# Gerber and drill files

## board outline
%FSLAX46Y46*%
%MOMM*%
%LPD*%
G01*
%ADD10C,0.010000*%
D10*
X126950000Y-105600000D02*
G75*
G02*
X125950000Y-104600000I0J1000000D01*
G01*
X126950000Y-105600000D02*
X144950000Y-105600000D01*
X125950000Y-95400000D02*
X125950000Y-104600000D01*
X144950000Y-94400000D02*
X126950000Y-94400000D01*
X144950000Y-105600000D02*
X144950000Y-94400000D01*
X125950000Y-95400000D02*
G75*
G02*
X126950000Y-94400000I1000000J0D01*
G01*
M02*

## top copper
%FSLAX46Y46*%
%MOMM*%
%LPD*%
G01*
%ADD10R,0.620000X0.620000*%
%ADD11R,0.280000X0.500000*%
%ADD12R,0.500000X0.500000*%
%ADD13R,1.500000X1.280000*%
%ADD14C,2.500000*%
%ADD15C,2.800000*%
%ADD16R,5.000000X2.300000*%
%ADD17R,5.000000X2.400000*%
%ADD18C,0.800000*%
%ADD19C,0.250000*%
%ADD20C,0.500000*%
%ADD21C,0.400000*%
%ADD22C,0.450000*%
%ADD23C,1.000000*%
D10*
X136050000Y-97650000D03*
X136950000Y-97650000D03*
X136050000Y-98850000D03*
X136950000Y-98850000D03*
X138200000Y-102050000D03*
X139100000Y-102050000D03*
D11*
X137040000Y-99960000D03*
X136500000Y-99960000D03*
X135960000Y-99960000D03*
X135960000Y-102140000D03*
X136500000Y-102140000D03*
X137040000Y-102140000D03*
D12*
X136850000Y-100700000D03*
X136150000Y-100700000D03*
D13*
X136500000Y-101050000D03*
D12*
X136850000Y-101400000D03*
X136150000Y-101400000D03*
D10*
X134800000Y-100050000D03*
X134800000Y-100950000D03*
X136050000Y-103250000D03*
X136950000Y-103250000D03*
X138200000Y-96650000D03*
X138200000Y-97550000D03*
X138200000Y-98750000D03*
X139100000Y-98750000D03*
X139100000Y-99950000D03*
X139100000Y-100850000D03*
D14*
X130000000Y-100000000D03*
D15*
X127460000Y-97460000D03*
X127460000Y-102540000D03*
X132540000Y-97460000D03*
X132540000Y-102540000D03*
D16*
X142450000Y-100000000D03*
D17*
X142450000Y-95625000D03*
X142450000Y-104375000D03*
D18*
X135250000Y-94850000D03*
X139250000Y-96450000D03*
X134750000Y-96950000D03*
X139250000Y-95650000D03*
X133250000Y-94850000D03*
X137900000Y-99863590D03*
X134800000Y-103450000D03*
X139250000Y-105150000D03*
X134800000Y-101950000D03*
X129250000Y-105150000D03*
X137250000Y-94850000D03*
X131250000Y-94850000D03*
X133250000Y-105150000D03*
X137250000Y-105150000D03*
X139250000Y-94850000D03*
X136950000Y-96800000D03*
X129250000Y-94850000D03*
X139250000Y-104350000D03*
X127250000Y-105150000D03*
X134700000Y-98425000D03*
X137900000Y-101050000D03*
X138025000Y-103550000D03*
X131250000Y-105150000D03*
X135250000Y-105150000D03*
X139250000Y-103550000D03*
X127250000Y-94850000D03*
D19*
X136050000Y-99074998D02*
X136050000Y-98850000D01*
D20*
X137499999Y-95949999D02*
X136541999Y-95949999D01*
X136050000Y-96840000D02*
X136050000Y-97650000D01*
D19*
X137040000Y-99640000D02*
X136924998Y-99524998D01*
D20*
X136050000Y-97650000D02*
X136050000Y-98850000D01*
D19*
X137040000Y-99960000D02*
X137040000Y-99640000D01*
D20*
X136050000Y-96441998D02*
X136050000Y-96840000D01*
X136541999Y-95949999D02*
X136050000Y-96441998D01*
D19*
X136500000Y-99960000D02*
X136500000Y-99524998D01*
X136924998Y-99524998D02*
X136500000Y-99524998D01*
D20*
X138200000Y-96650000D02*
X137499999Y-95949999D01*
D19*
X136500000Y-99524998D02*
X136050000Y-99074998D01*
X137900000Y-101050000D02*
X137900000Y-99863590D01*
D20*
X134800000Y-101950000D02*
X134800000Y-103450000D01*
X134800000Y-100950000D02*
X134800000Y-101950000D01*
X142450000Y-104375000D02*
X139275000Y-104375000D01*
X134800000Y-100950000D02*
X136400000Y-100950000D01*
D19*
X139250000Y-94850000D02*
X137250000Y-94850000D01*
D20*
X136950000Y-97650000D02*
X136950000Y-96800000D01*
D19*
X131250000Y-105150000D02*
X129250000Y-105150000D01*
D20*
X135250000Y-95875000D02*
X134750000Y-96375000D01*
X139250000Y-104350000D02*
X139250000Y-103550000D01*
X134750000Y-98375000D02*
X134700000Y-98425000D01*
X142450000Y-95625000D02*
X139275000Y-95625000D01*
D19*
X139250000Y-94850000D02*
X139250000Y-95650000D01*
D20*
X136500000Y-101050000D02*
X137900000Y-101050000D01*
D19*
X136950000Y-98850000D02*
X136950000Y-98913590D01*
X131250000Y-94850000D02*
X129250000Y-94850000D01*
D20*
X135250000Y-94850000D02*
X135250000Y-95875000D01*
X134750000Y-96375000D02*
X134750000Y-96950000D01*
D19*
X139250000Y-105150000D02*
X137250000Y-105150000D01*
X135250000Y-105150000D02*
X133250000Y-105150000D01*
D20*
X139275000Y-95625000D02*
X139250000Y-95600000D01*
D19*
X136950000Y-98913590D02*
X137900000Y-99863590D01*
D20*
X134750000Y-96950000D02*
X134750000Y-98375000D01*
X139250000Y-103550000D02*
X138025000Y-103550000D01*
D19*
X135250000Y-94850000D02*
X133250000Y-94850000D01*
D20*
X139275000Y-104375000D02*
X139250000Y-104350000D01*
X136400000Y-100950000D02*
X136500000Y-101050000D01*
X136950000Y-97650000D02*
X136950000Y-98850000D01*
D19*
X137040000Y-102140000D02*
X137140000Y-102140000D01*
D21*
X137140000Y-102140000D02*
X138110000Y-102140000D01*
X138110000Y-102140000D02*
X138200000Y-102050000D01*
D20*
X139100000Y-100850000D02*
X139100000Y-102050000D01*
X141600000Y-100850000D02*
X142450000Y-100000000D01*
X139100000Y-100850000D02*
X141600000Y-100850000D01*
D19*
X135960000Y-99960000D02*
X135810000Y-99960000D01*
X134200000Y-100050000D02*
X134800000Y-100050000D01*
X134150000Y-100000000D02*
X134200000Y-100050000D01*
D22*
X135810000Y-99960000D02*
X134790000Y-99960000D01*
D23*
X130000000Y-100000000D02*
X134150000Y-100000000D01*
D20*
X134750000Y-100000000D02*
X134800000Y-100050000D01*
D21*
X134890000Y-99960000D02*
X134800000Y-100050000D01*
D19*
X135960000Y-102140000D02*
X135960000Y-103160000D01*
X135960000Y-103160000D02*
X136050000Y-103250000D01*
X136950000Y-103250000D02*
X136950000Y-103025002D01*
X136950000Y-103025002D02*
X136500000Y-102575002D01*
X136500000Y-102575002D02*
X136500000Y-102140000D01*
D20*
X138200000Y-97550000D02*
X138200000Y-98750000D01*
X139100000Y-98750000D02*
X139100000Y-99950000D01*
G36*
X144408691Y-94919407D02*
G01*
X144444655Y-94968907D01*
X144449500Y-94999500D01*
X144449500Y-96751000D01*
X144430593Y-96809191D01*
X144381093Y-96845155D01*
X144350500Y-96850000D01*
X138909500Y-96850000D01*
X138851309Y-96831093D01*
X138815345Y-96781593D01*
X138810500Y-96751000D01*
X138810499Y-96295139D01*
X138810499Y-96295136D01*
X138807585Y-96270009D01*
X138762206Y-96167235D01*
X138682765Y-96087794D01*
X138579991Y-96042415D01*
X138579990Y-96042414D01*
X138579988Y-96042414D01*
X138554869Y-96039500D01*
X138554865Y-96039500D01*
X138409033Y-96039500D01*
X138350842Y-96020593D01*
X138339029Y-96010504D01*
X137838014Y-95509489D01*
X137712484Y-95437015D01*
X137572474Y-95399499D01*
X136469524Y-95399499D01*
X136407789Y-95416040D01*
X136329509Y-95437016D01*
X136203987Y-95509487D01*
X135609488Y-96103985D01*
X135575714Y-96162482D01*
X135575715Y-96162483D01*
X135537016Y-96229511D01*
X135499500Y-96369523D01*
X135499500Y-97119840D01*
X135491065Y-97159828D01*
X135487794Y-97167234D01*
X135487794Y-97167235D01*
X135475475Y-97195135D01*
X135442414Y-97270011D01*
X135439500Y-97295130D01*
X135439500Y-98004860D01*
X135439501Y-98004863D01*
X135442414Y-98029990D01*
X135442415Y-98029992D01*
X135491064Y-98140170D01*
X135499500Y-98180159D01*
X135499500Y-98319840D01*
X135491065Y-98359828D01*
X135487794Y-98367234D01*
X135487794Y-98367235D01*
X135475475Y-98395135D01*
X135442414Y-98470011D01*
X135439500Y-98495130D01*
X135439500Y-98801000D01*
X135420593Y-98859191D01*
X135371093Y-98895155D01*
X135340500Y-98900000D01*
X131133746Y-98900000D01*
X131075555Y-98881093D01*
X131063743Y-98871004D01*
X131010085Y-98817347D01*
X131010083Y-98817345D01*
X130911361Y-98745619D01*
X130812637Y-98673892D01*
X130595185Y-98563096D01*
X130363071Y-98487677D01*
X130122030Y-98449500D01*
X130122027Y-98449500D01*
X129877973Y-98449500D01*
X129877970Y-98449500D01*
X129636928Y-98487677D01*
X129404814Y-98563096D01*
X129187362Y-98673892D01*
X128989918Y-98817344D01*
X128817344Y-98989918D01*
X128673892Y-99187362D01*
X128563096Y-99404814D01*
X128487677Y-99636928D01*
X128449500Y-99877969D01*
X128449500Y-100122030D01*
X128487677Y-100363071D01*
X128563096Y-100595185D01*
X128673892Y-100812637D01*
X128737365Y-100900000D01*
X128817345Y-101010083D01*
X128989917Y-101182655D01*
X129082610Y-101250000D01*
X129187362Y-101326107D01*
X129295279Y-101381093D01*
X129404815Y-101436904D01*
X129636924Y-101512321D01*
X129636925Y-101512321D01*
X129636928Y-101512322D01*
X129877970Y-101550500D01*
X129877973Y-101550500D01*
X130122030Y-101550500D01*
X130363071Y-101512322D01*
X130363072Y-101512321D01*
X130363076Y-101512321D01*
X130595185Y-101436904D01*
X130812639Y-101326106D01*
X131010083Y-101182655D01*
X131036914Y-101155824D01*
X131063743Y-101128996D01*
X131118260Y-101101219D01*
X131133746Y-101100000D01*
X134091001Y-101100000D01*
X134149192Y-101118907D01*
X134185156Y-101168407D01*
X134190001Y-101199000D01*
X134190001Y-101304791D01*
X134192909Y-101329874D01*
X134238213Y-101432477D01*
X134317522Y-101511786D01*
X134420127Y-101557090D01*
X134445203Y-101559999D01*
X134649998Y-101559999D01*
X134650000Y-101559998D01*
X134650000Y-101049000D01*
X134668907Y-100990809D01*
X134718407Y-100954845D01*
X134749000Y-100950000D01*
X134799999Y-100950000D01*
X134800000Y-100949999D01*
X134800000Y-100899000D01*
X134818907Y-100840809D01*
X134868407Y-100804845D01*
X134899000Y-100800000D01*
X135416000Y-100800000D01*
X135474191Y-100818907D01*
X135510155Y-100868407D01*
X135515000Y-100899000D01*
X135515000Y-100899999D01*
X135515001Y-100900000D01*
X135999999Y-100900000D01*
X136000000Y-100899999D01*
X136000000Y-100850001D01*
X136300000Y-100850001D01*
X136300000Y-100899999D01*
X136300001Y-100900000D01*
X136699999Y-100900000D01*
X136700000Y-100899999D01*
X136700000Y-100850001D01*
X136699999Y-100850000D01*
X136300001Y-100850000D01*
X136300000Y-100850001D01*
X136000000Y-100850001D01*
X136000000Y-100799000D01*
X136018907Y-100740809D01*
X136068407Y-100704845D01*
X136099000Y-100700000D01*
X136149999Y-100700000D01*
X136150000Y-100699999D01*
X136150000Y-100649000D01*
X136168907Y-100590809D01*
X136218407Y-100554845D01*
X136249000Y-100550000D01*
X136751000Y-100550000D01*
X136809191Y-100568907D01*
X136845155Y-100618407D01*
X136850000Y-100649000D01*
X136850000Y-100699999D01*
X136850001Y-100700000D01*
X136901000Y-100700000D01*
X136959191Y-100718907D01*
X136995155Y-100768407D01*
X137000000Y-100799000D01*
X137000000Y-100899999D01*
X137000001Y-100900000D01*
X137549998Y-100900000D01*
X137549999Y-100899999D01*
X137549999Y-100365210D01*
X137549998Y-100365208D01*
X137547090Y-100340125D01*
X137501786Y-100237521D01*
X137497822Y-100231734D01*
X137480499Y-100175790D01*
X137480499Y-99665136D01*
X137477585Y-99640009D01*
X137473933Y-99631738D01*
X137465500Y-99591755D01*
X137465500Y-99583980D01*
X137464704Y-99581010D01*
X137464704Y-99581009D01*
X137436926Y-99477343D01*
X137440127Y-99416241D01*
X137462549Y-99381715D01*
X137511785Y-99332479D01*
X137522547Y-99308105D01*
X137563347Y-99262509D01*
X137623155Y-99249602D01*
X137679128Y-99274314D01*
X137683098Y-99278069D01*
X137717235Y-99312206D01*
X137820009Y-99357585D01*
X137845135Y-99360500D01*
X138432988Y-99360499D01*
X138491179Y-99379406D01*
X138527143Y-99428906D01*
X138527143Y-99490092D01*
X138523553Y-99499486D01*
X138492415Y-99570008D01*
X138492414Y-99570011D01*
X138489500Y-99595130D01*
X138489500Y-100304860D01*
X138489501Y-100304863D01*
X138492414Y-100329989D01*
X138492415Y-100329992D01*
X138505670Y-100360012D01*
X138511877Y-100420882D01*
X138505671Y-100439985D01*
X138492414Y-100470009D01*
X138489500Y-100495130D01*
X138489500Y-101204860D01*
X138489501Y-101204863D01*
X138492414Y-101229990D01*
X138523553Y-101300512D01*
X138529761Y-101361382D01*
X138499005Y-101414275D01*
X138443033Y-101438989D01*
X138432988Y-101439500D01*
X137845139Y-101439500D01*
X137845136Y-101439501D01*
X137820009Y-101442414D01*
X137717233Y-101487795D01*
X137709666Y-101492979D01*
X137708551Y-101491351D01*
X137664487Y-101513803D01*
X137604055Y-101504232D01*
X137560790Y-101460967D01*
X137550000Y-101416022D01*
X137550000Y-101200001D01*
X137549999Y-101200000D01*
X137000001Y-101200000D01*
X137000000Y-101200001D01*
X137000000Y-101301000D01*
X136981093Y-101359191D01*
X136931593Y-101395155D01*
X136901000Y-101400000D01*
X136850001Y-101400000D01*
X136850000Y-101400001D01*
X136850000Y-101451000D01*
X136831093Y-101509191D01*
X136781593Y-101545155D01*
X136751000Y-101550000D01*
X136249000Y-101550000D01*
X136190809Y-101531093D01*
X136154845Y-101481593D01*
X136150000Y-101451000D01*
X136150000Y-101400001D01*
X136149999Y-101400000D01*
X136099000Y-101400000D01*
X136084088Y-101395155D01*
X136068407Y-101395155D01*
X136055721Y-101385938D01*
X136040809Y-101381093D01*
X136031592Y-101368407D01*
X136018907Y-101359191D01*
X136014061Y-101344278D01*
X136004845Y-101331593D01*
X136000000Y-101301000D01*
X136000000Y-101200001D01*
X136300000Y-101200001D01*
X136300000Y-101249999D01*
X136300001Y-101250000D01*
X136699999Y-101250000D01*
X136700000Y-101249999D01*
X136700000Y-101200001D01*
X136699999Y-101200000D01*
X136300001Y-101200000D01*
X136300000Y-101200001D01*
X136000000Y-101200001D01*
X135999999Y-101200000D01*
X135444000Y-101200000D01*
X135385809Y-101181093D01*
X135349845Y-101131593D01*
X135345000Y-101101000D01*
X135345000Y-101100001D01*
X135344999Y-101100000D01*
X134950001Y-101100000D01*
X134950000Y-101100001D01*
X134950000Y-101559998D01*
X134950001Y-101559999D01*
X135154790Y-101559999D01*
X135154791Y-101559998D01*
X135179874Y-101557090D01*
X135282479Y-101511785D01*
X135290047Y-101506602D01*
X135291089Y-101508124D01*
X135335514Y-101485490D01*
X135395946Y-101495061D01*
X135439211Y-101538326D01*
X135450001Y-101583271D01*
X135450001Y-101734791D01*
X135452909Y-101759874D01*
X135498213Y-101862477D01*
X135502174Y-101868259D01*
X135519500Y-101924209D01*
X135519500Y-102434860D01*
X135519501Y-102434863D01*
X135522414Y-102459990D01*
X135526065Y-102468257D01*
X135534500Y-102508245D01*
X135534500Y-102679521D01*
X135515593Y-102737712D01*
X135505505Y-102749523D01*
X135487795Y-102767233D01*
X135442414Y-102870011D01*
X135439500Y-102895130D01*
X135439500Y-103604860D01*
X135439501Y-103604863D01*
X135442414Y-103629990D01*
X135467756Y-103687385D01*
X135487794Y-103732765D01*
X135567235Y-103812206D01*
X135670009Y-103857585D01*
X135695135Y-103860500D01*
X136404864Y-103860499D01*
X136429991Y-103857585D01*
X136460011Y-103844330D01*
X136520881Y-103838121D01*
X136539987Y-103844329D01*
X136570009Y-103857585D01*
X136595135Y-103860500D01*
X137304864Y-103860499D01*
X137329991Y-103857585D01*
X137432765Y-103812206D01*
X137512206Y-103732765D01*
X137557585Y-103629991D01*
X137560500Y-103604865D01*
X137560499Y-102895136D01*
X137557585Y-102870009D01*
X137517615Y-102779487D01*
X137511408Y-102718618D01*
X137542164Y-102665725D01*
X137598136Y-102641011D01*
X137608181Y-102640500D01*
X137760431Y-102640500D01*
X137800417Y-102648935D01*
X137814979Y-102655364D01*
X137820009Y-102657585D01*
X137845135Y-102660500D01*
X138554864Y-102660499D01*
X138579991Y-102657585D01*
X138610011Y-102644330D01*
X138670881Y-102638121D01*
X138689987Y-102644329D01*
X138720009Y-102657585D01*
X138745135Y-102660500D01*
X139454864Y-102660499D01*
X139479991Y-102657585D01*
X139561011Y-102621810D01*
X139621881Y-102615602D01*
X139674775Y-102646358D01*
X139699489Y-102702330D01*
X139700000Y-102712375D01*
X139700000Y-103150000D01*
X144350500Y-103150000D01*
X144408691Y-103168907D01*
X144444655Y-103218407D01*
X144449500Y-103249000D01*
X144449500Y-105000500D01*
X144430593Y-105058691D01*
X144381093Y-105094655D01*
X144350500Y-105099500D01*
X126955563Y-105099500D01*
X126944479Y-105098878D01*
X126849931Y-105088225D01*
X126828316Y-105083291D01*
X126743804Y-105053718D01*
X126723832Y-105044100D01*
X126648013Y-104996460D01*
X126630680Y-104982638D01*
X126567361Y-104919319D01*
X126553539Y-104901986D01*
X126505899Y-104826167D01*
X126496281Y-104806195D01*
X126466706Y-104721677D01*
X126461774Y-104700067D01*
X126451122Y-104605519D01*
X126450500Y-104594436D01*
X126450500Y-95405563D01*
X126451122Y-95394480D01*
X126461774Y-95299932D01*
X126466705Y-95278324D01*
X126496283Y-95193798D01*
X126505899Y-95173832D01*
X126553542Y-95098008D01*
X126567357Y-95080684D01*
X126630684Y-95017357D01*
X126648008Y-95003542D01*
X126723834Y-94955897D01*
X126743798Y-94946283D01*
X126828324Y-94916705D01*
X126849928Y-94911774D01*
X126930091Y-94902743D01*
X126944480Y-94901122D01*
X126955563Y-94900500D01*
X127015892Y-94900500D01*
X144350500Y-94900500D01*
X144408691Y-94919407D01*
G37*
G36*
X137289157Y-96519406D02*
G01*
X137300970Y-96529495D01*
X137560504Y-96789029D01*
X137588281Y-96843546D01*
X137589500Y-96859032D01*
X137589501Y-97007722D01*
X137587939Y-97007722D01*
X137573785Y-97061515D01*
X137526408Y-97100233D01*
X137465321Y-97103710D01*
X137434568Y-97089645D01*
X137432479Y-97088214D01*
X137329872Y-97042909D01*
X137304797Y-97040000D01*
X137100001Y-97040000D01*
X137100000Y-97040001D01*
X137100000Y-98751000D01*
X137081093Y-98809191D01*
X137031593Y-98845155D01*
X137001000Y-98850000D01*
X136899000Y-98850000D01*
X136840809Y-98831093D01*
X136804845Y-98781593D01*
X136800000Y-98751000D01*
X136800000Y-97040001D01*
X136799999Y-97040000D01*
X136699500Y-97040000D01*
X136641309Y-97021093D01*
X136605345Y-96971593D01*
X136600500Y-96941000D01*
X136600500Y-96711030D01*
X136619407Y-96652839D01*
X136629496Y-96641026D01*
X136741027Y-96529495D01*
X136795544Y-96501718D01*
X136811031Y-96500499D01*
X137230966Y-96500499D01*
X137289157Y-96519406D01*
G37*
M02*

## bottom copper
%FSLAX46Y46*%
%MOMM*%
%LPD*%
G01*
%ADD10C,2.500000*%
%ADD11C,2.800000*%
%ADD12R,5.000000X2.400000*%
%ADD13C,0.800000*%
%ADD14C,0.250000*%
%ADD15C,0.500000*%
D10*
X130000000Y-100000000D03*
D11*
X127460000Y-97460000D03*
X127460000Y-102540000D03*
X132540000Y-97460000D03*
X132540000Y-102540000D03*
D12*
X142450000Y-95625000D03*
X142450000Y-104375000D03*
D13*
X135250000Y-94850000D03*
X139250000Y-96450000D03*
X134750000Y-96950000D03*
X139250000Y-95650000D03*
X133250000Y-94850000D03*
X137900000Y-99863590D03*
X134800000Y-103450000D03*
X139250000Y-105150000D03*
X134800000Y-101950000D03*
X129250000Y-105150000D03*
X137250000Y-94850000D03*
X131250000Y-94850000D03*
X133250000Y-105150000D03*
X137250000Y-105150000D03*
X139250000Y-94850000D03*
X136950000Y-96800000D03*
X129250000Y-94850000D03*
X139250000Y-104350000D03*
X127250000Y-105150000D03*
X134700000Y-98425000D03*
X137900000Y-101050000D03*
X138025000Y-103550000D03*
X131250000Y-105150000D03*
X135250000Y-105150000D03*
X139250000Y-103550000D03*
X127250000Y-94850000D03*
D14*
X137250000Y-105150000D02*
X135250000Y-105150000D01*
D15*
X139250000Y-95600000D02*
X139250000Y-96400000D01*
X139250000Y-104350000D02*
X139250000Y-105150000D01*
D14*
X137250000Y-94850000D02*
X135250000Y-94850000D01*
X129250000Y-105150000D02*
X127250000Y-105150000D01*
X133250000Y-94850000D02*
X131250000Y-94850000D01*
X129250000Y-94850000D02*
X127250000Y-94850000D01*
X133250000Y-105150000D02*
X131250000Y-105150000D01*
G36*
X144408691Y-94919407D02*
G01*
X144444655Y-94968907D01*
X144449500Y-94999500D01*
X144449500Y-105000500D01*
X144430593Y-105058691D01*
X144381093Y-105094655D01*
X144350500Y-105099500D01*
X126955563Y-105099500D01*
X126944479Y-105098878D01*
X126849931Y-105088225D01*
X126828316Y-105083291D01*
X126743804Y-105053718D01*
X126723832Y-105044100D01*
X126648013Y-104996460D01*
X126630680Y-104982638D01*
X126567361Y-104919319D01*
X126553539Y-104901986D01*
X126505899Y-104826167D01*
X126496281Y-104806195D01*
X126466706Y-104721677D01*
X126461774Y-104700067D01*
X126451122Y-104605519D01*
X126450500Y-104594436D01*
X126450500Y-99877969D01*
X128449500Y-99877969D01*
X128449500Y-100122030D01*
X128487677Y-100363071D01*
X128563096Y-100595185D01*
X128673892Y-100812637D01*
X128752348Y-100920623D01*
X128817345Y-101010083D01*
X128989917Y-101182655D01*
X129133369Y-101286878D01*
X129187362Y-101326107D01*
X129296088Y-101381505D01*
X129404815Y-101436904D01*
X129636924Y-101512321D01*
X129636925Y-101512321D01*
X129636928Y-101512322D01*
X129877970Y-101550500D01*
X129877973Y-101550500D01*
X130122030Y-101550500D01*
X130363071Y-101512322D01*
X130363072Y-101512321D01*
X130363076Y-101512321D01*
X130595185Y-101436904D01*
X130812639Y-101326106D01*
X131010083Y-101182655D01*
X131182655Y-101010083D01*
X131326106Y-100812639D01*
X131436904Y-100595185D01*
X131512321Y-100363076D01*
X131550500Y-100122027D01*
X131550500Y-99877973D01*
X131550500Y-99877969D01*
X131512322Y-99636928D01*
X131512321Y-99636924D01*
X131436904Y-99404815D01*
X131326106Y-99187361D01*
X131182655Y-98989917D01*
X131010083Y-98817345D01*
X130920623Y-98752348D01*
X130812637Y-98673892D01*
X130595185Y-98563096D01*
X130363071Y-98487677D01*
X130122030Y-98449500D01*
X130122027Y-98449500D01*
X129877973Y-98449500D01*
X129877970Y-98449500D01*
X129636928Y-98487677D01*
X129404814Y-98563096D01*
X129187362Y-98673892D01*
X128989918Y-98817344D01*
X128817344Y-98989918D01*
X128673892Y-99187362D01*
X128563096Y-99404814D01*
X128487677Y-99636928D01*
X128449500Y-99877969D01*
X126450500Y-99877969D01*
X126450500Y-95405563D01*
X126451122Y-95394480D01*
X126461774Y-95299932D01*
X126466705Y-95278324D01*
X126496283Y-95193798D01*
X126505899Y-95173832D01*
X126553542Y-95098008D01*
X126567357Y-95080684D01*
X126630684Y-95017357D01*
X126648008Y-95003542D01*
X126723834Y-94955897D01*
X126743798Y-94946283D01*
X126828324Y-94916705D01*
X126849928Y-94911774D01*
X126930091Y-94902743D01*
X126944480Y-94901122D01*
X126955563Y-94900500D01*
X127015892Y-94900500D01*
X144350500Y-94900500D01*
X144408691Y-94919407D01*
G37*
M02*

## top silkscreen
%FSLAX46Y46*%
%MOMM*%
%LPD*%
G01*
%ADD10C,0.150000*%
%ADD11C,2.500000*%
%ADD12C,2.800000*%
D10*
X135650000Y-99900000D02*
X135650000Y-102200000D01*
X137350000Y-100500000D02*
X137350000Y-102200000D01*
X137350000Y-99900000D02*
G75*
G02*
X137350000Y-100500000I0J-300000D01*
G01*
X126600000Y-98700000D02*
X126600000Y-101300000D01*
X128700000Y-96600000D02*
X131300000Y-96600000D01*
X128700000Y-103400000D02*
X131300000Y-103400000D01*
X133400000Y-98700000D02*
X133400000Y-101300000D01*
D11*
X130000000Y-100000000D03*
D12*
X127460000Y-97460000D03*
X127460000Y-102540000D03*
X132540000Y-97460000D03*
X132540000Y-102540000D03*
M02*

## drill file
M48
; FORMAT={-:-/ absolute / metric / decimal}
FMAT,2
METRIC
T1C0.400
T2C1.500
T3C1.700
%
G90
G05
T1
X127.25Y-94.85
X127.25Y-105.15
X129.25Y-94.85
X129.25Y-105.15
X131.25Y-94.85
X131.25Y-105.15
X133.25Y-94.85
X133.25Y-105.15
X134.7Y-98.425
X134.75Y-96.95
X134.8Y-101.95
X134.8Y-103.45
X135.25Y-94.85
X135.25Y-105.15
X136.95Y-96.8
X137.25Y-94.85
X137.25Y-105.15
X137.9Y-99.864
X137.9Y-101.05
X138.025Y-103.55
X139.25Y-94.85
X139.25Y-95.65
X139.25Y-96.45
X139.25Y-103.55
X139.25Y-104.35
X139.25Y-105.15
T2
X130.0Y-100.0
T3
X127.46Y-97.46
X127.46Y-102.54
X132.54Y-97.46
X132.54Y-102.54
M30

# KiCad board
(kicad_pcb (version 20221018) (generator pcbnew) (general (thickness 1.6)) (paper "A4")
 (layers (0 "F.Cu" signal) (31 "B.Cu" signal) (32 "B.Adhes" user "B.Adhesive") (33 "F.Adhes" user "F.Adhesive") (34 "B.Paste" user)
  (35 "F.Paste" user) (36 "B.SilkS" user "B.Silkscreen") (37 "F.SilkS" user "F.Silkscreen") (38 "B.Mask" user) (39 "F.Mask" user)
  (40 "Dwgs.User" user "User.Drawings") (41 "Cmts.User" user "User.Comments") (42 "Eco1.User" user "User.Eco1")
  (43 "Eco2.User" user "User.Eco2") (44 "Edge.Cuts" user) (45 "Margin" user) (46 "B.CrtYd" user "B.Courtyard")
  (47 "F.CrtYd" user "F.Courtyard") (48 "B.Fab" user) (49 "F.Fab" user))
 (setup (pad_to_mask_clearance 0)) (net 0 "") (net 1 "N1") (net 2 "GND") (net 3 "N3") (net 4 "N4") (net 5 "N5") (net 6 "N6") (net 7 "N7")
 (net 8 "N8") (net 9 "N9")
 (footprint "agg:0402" (layer "F.Cu") (at 136.5 97.65)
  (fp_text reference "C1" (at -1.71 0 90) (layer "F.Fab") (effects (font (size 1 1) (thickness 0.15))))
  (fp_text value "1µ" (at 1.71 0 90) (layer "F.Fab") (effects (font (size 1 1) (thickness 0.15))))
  (pad "1" smd rect (at -0.45 0) (size 0.62 0.62) (layers "F.Cu" "F.Paste" "F.Mask") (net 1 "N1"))
  (pad "2" smd rect (at 0.45 0) (size 0.62 0.62) (layers "F.Cu" "F.Paste" "F.Mask") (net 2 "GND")))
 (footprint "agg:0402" (layer "F.Cu") (at 136.5 98.85)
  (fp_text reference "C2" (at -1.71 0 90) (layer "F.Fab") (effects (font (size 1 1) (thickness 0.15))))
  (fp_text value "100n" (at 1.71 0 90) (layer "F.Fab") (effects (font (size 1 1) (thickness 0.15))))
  (pad "1" smd rect (at -0.45 0) (size 0.62 0.62) (layers "F.Cu" "F.Paste" "F.Mask") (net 1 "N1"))
  (pad "2" smd rect (at 0.45 0) (size 0.62 0.62) (layers "F.Cu" "F.Paste" "F.Mask") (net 2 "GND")))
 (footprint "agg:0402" (layer "F.Cu") (at 138.65 102.05)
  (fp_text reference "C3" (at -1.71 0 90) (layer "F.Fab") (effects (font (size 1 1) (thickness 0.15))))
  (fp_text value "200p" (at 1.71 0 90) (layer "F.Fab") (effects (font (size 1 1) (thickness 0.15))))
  (pad "1" smd rect (at -0.45 0) (size 0.62 0.62) (layers "F.Cu" "F.Paste" "F.Mask") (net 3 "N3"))
  (pad "2" smd rect (at 0.45 0) (size 0.62 0.62) (layers "F.Cu" "F.Paste" "F.Mask") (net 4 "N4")))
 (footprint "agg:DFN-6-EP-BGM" (layer "F.Cu") (at 136.5 101.05 -90)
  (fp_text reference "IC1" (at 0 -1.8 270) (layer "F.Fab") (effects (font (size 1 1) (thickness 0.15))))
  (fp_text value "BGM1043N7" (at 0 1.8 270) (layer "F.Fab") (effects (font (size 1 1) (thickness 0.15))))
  (fp_line (start -1.15 0.85) (end 1.15 0.85) (stroke (width 0.15) (type solid)) (layer "F.SilkS"))
  (fp_line (start -0.55 -0.85) (end 1.15 -0.85) (stroke (width 0.15) (type solid)) (layer "F.SilkS"))
  (fp_arc (start -1.15 -0.85) (mid -0.85 -1.15) (end -0.55 -0.85) (stroke (width 0.15) (type solid)) (layer "F.SilkS"))
  (pad "1" smd rect (at -1.09 -0.54 270) (size 0.5 0.28) (layers "F.Cu" "F.Paste" "F.Mask") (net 1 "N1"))
  (pad "2" smd rect (at -1.09 0 270) (size 0.5 0.28) (layers "F.Cu" "F.Paste" "F.Mask") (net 1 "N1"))
  (pad "3" smd rect (at -1.09 0.54 270) (size 0.5 0.28) (layers "F.Cu" "F.Paste" "F.Mask") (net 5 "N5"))
  (pad "4" smd rect (at 1.09 0.54 270) (size 0.5 0.28) (layers "F.Cu" "F.Paste" "F.Mask") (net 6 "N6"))
  (pad "5" smd rect (at 1.09 0 270) (size 0.5 0.28) (layers "F.Cu" "F.Paste" "F.Mask") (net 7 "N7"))
  (pad "6" smd rect (at 1.09 -0.54 270) (size 0.5 0.28) (layers "F.Cu" "F.Paste" "F.Mask") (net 3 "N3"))
  (pad "EP" smd rect (at -0.35 -0.35 270) (size 0.5 0.5) (layers "F.Cu" "F.Paste") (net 2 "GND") (solder_paste_margin 0.001))
  (pad "EP" smd rect (at -0.35 0.35 270) (size 0.5 0.5) (layers "F.Cu" "F.Paste") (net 2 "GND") (solder_paste_margin 0.001))
  (pad "EP" smd rect (at 0 0 270) (size 1.28 1.5) (layers "F.Cu" "F.Mask") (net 2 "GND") (solder_mask_margin 0.001))
  (pad "EP" smd rect (at 0.35 -0.35 270) (size 0.5 0.5) (layers "F.Cu" "F.Paste") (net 2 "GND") (solder_paste_margin 0.001))
  (pad "EP" smd rect (at 0.35 0.35 270) (size 0.5 0.5) (layers "F.Cu" "F.Paste") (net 2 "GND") (solder_paste_margin 0.001)))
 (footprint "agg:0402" (layer "F.Cu") (at 134.8 100.5 -90)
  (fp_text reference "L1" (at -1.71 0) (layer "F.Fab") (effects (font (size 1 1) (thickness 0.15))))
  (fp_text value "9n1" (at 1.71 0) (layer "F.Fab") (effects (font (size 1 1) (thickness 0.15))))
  (pad "1" smd rect (at -0.45 0 270) (size 0.62 0.62) (layers "F.Cu" "F.Paste" "F.Mask") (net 5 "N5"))
  (pad "2" smd rect (at 0.45 0 270) (size 0.62 0.62) (layers "F.Cu" "F.Paste" "F.Mask") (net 2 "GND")))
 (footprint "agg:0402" (layer "F.Cu") (at 136.5 103.25)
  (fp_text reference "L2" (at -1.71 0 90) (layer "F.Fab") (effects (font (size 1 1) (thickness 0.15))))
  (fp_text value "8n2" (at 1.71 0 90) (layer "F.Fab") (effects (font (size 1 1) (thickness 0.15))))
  (pad "1" smd rect (at -0.45 0) (size 0.62 0.62) (layers "F.Cu" "F.Paste" "F.Mask") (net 6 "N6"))
  (pad "2" smd rect (at 0.45 0) (size 0.62 0.62) (layers "F.Cu" "F.Paste" "F.Mask") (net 7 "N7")))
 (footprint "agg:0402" (layer "F.Cu") (at 138.2 97.1 -90)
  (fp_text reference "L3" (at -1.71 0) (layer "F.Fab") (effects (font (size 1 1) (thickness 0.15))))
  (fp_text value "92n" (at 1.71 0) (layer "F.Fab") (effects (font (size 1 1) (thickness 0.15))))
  (pad "1" smd rect (at -0.45 0 270) (size 0.62 0.62) (layers "F.Cu" "F.Paste" "F.Mask") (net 1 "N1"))
  (pad "2" smd rect (at 0.45 0 270) (size 0.62 0.62) (layers "F.Cu" "F.Paste" "F.Mask") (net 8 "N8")))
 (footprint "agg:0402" (layer "F.Cu") (at 138.65 98.75)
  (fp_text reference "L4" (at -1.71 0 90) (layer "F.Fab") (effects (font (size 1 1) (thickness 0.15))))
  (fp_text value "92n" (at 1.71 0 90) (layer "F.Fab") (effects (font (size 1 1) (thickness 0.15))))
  (pad "1" smd rect (at -0.45 0) (size 0.62 0.62) (layers "F.Cu" "F.Paste" "F.Mask") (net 8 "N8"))
  (pad "2" smd rect (at 0.45 0) (size 0.62 0.62) (layers "F.Cu" "F.Paste" "F.Mask") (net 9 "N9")))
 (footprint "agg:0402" (layer "F.Cu") (at 139.1 100.4 -90)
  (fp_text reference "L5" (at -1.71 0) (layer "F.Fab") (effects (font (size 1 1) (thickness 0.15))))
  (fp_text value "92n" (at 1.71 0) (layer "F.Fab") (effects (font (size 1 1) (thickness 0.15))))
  (pad "1" smd rect (at -0.45 0 270) (size 0.62 0.62) (layers "F.Cu" "F.Paste" "F.Mask") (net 9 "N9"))
  (pad "2" smd rect (at 0.45 0 270) (size 0.62 0.62) (layers "F.Cu" "F.Paste" "F.Mask") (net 4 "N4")))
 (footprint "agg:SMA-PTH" (layer "F.Cu") (at 130 100)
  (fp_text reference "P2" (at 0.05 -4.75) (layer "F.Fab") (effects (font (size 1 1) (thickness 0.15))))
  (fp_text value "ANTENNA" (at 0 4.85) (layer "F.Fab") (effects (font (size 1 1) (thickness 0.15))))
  (fp_line (start -3.4 -1.3) (end -3.4 1.3) (stroke (width 0.15) (type solid)) (layer "F.SilkS"))
  (fp_line (start -1.3 -3.4) (end 1.3 -3.4) (stroke (width 0.15) (type solid)) (layer "F.SilkS"))
  (fp_line (start -1.3 3.4) (end 1.3 3.4) (stroke (width 0.15) (type solid)) (layer "F.SilkS"))
  (fp_line (start 3.4 -1.3) (end 3.4 1.3) (stroke (width 0.15) (type solid)) (layer "F.SilkS"))
  (pad "1" thru_hole circle (at 0 0) (size 2.5 2.5) (drill 1.5) (layers "*.Cu" "*.Mask" "F.SilkS") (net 5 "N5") (zone_connect 2))
  (pad "2" thru_hole circle (at -2.54 -2.54) (size 2.8 2.8) (drill 1.7) (layers "*.Cu" "*.Mask" "F.SilkS") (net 2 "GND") (zone_connect 2))
  (pad "2" thru_hole circle (at -2.54 2.54) (size 2.8 2.8) (drill 1.7) (layers "*.Cu" "*.Mask" "F.SilkS") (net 2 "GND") (zone_connect 2))
  (pad "2" thru_hole circle (at 2.54 -2.54) (size 2.8 2.8) (drill 1.7) (layers "*.Cu" "*.Mask" "F.SilkS") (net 2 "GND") (zone_connect 2))
  (pad "2" thru_hole circle (at 2.54 2.54) (size 2.8 2.8) (drill 1.7) (layers "*.Cu" "*.Mask" "F.SilkS") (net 2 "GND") (zone_connect 2)))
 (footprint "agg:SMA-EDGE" (layer "F.Cu") (at 142.45 100 -90)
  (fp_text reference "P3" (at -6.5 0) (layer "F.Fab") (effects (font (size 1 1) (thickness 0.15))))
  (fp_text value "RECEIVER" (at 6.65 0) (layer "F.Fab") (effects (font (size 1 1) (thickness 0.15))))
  (pad "1" smd rect (at 0 0 270) (size 2.3 5) (layers "F.Cu" "F.Paste" "F.Mask") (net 4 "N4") (zone_connect 2))
  (pad "2" smd rect (at -4.375 0 270) (size 2.4 5) (layers "F.Cu" "F.Paste" "F.Mask") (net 2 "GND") (zone_connect 2))
  (pad "2" smd rect (at -4.375 0 270) (size 2.4 5) (layers "B.Cu" "B.Paste" "B.Mask") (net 2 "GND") (zone_connect 2))
  (pad "2" smd rect (at 4.375 0 270) (size 2.4 5) (layers "F.Cu" "F.Paste" "F.Mask") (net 2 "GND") (zone_connect 2))
  (pad "2" smd rect (at 4.375 0 270) (size 2.4 5) (layers "B.Cu" "B.Paste" "B.Mask") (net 2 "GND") (zone_connect 2)))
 (gr_arc (start 126.95 105.6) (mid 126.242893 105.307107) (end 125.95 104.6) (stroke (width 0.01) (type solid)) (layer "Edge.Cuts"))
 (gr_line (start 126.95 105.6) (end 144.95 105.6) (stroke (width 0.01) (type solid)) (layer "Edge.Cuts"))
 (gr_line (start 125.95 95.4) (end 125.95 104.6) (stroke (width 0.01) (type solid)) (layer "Edge.Cuts"))
 (gr_line (start 144.95 94.4) (end 126.95 94.4) (stroke (width 0.01) (type solid)) (layer "Edge.Cuts"))
 (gr_line (start 144.95 105.6) (end 144.95 94.4) (stroke (width 0.01) (type solid)) (layer "Edge.Cuts"))
 (gr_arc (start 125.95 95.4) (mid 126.242893 94.692893) (end 126.95 94.4) (stroke (width 0.01) (type solid)) (layer "Edge.Cuts"))
 (segment (start 136.05 99.074998) (end 136.05 98.85) (width 0.25) (layer "F.Cu") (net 1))
 (segment (start 137.499999 95.949999) (end 136.541999 95.949999) (width 0.5) (layer "F.Cu") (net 1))
 (segment (start 136.05 96.84) (end 136.05 97.65) (width 0.5) (layer "F.Cu") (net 1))
 (segment (start 137.04 99.64) (end 136.924998 99.524998) (width 0.25) (layer "F.Cu") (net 1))
 (segment (start 136.05 97.65) (end 136.05 98.85) (width 0.5) (layer "F.Cu") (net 1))
 (segment (start 137.04 99.96) (end 137.04 99.64) (width 0.25) (layer "F.Cu") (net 1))
 (segment (start 136.05 96.441998) (end 136.05 96.84) (width 0.5) (layer "F.Cu") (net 1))
 (segment (start 136.541999 95.949999) (end 136.05 96.441998) (width 0.5) (layer "F.Cu") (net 1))
 (segment (start 136.5 99.96) (end 136.5 99.524998) (width 0.25) (layer "F.Cu") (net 1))
 (segment (start 136.924998 99.524998) (end 136.5 99.524998) (width 0.25) (layer "F.Cu") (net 1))
 (segment (start 138.2 96.65) (end 137.499999 95.949999) (width 0.5) (layer "F.Cu") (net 1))
 (segment (start 136.5 99.524998) (end 136.05 99.074998) (width 0.25) (layer "F.Cu") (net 1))
 (segment (start 137.9 101.05) (end 137.9 99.86359) (width 0.25) (layer "F.Cu") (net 2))
 (segment (start 134.8 101.95) (end 134.8 103.45) (width 0.5) (layer "F.Cu") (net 2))
 (segment (start 134.8 100.95) (end 134.8 101.95) (width 0.5) (layer "F.Cu") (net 2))
 (segment (start 142.45 104.375) (end 139.275 104.375) (width 0.5) (layer "F.Cu") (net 2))
 (segment (start 134.8 100.95) (end 136.4 100.95) (width 0.5) (layer "F.Cu") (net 2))
 (segment (start 139.25 94.85) (end 137.25 94.85) (width 0.25) (layer "F.Cu") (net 2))
 (segment (start 136.95 97.65) (end 136.95 96.8) (width 0.5) (layer "F.Cu") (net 2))
 (segment (start 131.25 105.15) (end 129.25 105.15) (width 0.25) (layer "F.Cu") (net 2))
 (segment (start 135.25 95.875) (end 134.75 96.375) (width 0.5) (layer "F.Cu") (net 2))
 (segment (start 139.25 104.35) (end 139.25 103.55) (width 0.5) (layer "F.Cu") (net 2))
 (segment (start 134.75 98.375) (end 134.7 98.425) (width 0.5) (layer "F.Cu") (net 2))
 (segment (start 142.45 95.625) (end 139.275 95.625) (width 0.5) (layer "F.Cu") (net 2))
 (segment (start 139.25 94.85) (end 139.25 95.65) (width 0.25) (layer "F.Cu") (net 2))
 (segment (start 136.5 101.05) (end 137.9 101.05) (width 0.5) (layer "F.Cu") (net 2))
 (segment (start 136.95 98.85) (end 136.95 98.91359) (width 0.25) (layer "F.Cu") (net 2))
 (segment (start 131.25 94.85) (end 129.25 94.85) (width 0.25) (layer "F.Cu") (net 2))
 (segment (start 135.25 94.85) (end 135.25 95.875) (width 0.5) (layer "F.Cu") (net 2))
 (segment (start 134.75 96.375) (end 134.75 96.95) (width 0.5) (layer "F.Cu") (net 2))
 (segment (start 139.25 105.15) (end 137.25 105.15) (width 0.25) (layer "F.Cu") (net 2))
 (segment (start 135.25 105.15) (end 133.25 105.15) (width 0.25) (layer "F.Cu") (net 2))
 (segment (start 139.275 95.625) (end 139.25 95.6) (width 0.5) (layer "F.Cu") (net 2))
 (segment (start 136.95 98.91359) (end 137.9 99.86359) (width 0.25) (layer "F.Cu") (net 2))
 (segment (start 134.75 96.95) (end 134.75 98.375) (width 0.5) (layer "F.Cu") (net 2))
 (segment (start 139.25 103.55) (end 138.025 103.55) (width 0.5) (layer "F.Cu") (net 2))
 (segment (start 135.25 94.85) (end 133.25 94.85) (width 0.25) (layer "F.Cu") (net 2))
 (segment (start 139.275 104.375) (end 139.25 104.35) (width 0.5) (layer "F.Cu") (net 2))
 (segment (start 136.4 100.95) (end 136.5 101.05) (width 0.5) (layer "F.Cu") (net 2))
 (segment (start 136.95 97.65) (end 136.95 98.85) (width 0.5) (layer "F.Cu") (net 2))
 (via (at 135.25 94.85) (size 0.8) (drill 0.4) (layers "F.Cu" "B.Cu") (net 2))
 (via (at 139.25 96.45) (size 0.8) (drill 0.4) (layers "F.Cu" "B.Cu") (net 2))
 (via (at 134.75 96.95) (size 0.8) (drill 0.4) (layers "F.Cu" "B.Cu") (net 2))
 (via (at 139.25 95.65) (size 0.8) (drill 0.4) (layers "F.Cu" "B.Cu") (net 2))
 (via (at 133.25 94.85) (size 0.8) (drill 0.4) (layers "F.Cu" "B.Cu") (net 2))
 (via (at 137.9 99.86359) (size 0.8) (drill 0.4) (layers "F.Cu" "B.Cu") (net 2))
 (via (at 134.8 103.45) (size 0.8) (drill 0.4) (layers "F.Cu" "B.Cu") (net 2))
 (via (at 139.25 105.15) (size 0.8) (drill 0.4) (layers "F.Cu" "B.Cu") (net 2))
 (via (at 134.8 101.95) (size 0.8) (drill 0.4) (layers "F.Cu" "B.Cu") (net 2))
 (via (at 129.25 105.15) (size 0.8) (drill 0.4) (layers "F.Cu" "B.Cu") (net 2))
 (via (at 137.25 94.85) (size 0.8) (drill 0.4) (layers "F.Cu" "B.Cu") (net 2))
 (via (at 131.25 94.85) (size 0.8) (drill 0.4) (layers "F.Cu" "B.Cu") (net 2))
 (via (at 133.25 105.15) (size 0.8) (drill 0.4) (layers "F.Cu" "B.Cu") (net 2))
 (via (at 137.25 105.15) (size 0.8) (drill 0.4) (layers "F.Cu" "B.Cu") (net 2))
 (via (at 139.25 94.85) (size 0.8) (drill 0.4) (layers "F.Cu" "B.Cu") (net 2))
 (via (at 136.95 96.8) (size 0.8) (drill 0.4) (layers "F.Cu" "B.Cu") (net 2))
 (via (at 129.25 94.85) (size 0.8) (drill 0.4) (layers "F.Cu" "B.Cu") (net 2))
 (via (at 139.25 104.35) (size 0.8) (drill 0.4) (layers "F.Cu" "B.Cu") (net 2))
 (via (at 127.25 105.15) (size 0.8) (drill 0.4) (layers "F.Cu" "B.Cu") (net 2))
 (via (at 134.7 98.425) (size 0.8) (drill 0.4) (layers "F.Cu" "B.Cu") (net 2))
 (via (at 137.9 101.05) (size 0.8) (drill 0.4) (layers "F.Cu" "B.Cu") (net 2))
 (via (at 138.025 103.55) (size 0.8) (drill 0.4) (layers "F.Cu" "B.Cu") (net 2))
 (via (at 131.25 105.15) (size 0.8) (drill 0.4) (layers "F.Cu" "B.Cu") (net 2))
 (via (at 135.25 105.15) (size 0.8) (drill 0.4) (layers "F.Cu" "B.Cu") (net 2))
 (via (at 139.25 103.55) (size 0.8) (drill 0.4) (layers "F.Cu" "B.Cu") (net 2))
 (via (at 127.25 94.85) (size 0.8) (drill 0.4) (layers "F.Cu" "B.Cu") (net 2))
 (segment (start 137.25 105.15) (end 135.25 105.15) (width 0.25) (layer "B.Cu") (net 2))
 (segment (start 139.25 95.6) (end 139.25 96.4) (width 0.5) (layer "B.Cu") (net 2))
 (segment (start 139.25 104.35) (end 139.25 105.15) (width 0.5) (layer "B.Cu") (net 2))
 (segment (start 137.25 94.85) (end 135.25 94.85) (width 0.25) (layer "B.Cu") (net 2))
 (segment (start 129.25 105.15) (end 127.25 105.15) (width 0.25) (layer "B.Cu") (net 2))
 (segment (start 133.25 94.85) (end 131.25 94.85) (width 0.25) (layer "B.Cu") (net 2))
 (segment (start 129.25 94.85) (end 127.25 94.85) (width 0.25) (layer "B.Cu") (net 2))
 (segment (start 133.25 105.15) (end 131.25 105.15) (width 0.25) (layer "B.Cu") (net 2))
 (segment (start 137.04 102.14) (end 137.14 102.14) (width 0.25) (layer "F.Cu") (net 3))
 (segment (start 137.14 102.14) (end 138.11 102.14) (width 0.4) (layer "F.Cu") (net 3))
 (segment (start 138.11 102.14) (end 138.2 102.05) (width 0.4) (layer "F.Cu") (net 3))
 (segment (start 139.1 100.85) (end 139.1 102.05) (width 0.5) (layer "F.Cu") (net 4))
 (segment (start 141.6 100.85) (end 142.45 100) (width 0.5) (layer "F.Cu") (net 4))
 (segment (start 139.1 100.85) (end 141.6 100.85) (width 0.5) (layer "F.Cu") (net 4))
 (segment (start 135.96 99.96) (end 135.81 99.96) (width 0.25) (layer "F.Cu") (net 5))
 (segment (start 134.2 100.05) (end 134.8 100.05) (width 0.25) (layer "F.Cu") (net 5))
 (segment (start 134.15 100) (end 134.2 100.05) (width 0.25) (layer "F.Cu") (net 5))
 (segment (start 135.81 99.96) (end 134.79 99.96) (width 0.45) (layer "F.Cu") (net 5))
 (segment (start 130 100) (end 134.15 100) (width 1) (layer "F.Cu") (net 5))
 (segment (start 134.75 100) (end 134.8 100.05) (width 0.5) (layer "F.Cu") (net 5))
 (segment (start 134.89 99.96) (end 134.8 100.05) (width 0.4) (layer "F.Cu") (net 5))
 (segment (start 135.96 102.14) (end 135.96 103.16) (width 0.25) (layer "F.Cu") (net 6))
 (segment (start 135.96 103.16) (end 136.05 103.25) (width 0.25) (layer "F.Cu") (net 6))
 (segment (start 136.95 103.25) (end 136.95 103.025002) (width 0.25) (layer "F.Cu") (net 7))
 (segment (start 136.95 103.025002) (end 136.5 102.575002) (width 0.25) (layer "F.Cu") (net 7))
 (segment (start 136.5 102.575002) (end 136.5 102.14) (width 0.25) (layer "F.Cu") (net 7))
 (segment (start 138.2 97.55) (end 138.2 98.75) (width 0.5) (layer "F.Cu") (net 8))
 (segment (start 139.1 98.75) (end 139.1 99.95) (width 0.5) (layer "F.Cu") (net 9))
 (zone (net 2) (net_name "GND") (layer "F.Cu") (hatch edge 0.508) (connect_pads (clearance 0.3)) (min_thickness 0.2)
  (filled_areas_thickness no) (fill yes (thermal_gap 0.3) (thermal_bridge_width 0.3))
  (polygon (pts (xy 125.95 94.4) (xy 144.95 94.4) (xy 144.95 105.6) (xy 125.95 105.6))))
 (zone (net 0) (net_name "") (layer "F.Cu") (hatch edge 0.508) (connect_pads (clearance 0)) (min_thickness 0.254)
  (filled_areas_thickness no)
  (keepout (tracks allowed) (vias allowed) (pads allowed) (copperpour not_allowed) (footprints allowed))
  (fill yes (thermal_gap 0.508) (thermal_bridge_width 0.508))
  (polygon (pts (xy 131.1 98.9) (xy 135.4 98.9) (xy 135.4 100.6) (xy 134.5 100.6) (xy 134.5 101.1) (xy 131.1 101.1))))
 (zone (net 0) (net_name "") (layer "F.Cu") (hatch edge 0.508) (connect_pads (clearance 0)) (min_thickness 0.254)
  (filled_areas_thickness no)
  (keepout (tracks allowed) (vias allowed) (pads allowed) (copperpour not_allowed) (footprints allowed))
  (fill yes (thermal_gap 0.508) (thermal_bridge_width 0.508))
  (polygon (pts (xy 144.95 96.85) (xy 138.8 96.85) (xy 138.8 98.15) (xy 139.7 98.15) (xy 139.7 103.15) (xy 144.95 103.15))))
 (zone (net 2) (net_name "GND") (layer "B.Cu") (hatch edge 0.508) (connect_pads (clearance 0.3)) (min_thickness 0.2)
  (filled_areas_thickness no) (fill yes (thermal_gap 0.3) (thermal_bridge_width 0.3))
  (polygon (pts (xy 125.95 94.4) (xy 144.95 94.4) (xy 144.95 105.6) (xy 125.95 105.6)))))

